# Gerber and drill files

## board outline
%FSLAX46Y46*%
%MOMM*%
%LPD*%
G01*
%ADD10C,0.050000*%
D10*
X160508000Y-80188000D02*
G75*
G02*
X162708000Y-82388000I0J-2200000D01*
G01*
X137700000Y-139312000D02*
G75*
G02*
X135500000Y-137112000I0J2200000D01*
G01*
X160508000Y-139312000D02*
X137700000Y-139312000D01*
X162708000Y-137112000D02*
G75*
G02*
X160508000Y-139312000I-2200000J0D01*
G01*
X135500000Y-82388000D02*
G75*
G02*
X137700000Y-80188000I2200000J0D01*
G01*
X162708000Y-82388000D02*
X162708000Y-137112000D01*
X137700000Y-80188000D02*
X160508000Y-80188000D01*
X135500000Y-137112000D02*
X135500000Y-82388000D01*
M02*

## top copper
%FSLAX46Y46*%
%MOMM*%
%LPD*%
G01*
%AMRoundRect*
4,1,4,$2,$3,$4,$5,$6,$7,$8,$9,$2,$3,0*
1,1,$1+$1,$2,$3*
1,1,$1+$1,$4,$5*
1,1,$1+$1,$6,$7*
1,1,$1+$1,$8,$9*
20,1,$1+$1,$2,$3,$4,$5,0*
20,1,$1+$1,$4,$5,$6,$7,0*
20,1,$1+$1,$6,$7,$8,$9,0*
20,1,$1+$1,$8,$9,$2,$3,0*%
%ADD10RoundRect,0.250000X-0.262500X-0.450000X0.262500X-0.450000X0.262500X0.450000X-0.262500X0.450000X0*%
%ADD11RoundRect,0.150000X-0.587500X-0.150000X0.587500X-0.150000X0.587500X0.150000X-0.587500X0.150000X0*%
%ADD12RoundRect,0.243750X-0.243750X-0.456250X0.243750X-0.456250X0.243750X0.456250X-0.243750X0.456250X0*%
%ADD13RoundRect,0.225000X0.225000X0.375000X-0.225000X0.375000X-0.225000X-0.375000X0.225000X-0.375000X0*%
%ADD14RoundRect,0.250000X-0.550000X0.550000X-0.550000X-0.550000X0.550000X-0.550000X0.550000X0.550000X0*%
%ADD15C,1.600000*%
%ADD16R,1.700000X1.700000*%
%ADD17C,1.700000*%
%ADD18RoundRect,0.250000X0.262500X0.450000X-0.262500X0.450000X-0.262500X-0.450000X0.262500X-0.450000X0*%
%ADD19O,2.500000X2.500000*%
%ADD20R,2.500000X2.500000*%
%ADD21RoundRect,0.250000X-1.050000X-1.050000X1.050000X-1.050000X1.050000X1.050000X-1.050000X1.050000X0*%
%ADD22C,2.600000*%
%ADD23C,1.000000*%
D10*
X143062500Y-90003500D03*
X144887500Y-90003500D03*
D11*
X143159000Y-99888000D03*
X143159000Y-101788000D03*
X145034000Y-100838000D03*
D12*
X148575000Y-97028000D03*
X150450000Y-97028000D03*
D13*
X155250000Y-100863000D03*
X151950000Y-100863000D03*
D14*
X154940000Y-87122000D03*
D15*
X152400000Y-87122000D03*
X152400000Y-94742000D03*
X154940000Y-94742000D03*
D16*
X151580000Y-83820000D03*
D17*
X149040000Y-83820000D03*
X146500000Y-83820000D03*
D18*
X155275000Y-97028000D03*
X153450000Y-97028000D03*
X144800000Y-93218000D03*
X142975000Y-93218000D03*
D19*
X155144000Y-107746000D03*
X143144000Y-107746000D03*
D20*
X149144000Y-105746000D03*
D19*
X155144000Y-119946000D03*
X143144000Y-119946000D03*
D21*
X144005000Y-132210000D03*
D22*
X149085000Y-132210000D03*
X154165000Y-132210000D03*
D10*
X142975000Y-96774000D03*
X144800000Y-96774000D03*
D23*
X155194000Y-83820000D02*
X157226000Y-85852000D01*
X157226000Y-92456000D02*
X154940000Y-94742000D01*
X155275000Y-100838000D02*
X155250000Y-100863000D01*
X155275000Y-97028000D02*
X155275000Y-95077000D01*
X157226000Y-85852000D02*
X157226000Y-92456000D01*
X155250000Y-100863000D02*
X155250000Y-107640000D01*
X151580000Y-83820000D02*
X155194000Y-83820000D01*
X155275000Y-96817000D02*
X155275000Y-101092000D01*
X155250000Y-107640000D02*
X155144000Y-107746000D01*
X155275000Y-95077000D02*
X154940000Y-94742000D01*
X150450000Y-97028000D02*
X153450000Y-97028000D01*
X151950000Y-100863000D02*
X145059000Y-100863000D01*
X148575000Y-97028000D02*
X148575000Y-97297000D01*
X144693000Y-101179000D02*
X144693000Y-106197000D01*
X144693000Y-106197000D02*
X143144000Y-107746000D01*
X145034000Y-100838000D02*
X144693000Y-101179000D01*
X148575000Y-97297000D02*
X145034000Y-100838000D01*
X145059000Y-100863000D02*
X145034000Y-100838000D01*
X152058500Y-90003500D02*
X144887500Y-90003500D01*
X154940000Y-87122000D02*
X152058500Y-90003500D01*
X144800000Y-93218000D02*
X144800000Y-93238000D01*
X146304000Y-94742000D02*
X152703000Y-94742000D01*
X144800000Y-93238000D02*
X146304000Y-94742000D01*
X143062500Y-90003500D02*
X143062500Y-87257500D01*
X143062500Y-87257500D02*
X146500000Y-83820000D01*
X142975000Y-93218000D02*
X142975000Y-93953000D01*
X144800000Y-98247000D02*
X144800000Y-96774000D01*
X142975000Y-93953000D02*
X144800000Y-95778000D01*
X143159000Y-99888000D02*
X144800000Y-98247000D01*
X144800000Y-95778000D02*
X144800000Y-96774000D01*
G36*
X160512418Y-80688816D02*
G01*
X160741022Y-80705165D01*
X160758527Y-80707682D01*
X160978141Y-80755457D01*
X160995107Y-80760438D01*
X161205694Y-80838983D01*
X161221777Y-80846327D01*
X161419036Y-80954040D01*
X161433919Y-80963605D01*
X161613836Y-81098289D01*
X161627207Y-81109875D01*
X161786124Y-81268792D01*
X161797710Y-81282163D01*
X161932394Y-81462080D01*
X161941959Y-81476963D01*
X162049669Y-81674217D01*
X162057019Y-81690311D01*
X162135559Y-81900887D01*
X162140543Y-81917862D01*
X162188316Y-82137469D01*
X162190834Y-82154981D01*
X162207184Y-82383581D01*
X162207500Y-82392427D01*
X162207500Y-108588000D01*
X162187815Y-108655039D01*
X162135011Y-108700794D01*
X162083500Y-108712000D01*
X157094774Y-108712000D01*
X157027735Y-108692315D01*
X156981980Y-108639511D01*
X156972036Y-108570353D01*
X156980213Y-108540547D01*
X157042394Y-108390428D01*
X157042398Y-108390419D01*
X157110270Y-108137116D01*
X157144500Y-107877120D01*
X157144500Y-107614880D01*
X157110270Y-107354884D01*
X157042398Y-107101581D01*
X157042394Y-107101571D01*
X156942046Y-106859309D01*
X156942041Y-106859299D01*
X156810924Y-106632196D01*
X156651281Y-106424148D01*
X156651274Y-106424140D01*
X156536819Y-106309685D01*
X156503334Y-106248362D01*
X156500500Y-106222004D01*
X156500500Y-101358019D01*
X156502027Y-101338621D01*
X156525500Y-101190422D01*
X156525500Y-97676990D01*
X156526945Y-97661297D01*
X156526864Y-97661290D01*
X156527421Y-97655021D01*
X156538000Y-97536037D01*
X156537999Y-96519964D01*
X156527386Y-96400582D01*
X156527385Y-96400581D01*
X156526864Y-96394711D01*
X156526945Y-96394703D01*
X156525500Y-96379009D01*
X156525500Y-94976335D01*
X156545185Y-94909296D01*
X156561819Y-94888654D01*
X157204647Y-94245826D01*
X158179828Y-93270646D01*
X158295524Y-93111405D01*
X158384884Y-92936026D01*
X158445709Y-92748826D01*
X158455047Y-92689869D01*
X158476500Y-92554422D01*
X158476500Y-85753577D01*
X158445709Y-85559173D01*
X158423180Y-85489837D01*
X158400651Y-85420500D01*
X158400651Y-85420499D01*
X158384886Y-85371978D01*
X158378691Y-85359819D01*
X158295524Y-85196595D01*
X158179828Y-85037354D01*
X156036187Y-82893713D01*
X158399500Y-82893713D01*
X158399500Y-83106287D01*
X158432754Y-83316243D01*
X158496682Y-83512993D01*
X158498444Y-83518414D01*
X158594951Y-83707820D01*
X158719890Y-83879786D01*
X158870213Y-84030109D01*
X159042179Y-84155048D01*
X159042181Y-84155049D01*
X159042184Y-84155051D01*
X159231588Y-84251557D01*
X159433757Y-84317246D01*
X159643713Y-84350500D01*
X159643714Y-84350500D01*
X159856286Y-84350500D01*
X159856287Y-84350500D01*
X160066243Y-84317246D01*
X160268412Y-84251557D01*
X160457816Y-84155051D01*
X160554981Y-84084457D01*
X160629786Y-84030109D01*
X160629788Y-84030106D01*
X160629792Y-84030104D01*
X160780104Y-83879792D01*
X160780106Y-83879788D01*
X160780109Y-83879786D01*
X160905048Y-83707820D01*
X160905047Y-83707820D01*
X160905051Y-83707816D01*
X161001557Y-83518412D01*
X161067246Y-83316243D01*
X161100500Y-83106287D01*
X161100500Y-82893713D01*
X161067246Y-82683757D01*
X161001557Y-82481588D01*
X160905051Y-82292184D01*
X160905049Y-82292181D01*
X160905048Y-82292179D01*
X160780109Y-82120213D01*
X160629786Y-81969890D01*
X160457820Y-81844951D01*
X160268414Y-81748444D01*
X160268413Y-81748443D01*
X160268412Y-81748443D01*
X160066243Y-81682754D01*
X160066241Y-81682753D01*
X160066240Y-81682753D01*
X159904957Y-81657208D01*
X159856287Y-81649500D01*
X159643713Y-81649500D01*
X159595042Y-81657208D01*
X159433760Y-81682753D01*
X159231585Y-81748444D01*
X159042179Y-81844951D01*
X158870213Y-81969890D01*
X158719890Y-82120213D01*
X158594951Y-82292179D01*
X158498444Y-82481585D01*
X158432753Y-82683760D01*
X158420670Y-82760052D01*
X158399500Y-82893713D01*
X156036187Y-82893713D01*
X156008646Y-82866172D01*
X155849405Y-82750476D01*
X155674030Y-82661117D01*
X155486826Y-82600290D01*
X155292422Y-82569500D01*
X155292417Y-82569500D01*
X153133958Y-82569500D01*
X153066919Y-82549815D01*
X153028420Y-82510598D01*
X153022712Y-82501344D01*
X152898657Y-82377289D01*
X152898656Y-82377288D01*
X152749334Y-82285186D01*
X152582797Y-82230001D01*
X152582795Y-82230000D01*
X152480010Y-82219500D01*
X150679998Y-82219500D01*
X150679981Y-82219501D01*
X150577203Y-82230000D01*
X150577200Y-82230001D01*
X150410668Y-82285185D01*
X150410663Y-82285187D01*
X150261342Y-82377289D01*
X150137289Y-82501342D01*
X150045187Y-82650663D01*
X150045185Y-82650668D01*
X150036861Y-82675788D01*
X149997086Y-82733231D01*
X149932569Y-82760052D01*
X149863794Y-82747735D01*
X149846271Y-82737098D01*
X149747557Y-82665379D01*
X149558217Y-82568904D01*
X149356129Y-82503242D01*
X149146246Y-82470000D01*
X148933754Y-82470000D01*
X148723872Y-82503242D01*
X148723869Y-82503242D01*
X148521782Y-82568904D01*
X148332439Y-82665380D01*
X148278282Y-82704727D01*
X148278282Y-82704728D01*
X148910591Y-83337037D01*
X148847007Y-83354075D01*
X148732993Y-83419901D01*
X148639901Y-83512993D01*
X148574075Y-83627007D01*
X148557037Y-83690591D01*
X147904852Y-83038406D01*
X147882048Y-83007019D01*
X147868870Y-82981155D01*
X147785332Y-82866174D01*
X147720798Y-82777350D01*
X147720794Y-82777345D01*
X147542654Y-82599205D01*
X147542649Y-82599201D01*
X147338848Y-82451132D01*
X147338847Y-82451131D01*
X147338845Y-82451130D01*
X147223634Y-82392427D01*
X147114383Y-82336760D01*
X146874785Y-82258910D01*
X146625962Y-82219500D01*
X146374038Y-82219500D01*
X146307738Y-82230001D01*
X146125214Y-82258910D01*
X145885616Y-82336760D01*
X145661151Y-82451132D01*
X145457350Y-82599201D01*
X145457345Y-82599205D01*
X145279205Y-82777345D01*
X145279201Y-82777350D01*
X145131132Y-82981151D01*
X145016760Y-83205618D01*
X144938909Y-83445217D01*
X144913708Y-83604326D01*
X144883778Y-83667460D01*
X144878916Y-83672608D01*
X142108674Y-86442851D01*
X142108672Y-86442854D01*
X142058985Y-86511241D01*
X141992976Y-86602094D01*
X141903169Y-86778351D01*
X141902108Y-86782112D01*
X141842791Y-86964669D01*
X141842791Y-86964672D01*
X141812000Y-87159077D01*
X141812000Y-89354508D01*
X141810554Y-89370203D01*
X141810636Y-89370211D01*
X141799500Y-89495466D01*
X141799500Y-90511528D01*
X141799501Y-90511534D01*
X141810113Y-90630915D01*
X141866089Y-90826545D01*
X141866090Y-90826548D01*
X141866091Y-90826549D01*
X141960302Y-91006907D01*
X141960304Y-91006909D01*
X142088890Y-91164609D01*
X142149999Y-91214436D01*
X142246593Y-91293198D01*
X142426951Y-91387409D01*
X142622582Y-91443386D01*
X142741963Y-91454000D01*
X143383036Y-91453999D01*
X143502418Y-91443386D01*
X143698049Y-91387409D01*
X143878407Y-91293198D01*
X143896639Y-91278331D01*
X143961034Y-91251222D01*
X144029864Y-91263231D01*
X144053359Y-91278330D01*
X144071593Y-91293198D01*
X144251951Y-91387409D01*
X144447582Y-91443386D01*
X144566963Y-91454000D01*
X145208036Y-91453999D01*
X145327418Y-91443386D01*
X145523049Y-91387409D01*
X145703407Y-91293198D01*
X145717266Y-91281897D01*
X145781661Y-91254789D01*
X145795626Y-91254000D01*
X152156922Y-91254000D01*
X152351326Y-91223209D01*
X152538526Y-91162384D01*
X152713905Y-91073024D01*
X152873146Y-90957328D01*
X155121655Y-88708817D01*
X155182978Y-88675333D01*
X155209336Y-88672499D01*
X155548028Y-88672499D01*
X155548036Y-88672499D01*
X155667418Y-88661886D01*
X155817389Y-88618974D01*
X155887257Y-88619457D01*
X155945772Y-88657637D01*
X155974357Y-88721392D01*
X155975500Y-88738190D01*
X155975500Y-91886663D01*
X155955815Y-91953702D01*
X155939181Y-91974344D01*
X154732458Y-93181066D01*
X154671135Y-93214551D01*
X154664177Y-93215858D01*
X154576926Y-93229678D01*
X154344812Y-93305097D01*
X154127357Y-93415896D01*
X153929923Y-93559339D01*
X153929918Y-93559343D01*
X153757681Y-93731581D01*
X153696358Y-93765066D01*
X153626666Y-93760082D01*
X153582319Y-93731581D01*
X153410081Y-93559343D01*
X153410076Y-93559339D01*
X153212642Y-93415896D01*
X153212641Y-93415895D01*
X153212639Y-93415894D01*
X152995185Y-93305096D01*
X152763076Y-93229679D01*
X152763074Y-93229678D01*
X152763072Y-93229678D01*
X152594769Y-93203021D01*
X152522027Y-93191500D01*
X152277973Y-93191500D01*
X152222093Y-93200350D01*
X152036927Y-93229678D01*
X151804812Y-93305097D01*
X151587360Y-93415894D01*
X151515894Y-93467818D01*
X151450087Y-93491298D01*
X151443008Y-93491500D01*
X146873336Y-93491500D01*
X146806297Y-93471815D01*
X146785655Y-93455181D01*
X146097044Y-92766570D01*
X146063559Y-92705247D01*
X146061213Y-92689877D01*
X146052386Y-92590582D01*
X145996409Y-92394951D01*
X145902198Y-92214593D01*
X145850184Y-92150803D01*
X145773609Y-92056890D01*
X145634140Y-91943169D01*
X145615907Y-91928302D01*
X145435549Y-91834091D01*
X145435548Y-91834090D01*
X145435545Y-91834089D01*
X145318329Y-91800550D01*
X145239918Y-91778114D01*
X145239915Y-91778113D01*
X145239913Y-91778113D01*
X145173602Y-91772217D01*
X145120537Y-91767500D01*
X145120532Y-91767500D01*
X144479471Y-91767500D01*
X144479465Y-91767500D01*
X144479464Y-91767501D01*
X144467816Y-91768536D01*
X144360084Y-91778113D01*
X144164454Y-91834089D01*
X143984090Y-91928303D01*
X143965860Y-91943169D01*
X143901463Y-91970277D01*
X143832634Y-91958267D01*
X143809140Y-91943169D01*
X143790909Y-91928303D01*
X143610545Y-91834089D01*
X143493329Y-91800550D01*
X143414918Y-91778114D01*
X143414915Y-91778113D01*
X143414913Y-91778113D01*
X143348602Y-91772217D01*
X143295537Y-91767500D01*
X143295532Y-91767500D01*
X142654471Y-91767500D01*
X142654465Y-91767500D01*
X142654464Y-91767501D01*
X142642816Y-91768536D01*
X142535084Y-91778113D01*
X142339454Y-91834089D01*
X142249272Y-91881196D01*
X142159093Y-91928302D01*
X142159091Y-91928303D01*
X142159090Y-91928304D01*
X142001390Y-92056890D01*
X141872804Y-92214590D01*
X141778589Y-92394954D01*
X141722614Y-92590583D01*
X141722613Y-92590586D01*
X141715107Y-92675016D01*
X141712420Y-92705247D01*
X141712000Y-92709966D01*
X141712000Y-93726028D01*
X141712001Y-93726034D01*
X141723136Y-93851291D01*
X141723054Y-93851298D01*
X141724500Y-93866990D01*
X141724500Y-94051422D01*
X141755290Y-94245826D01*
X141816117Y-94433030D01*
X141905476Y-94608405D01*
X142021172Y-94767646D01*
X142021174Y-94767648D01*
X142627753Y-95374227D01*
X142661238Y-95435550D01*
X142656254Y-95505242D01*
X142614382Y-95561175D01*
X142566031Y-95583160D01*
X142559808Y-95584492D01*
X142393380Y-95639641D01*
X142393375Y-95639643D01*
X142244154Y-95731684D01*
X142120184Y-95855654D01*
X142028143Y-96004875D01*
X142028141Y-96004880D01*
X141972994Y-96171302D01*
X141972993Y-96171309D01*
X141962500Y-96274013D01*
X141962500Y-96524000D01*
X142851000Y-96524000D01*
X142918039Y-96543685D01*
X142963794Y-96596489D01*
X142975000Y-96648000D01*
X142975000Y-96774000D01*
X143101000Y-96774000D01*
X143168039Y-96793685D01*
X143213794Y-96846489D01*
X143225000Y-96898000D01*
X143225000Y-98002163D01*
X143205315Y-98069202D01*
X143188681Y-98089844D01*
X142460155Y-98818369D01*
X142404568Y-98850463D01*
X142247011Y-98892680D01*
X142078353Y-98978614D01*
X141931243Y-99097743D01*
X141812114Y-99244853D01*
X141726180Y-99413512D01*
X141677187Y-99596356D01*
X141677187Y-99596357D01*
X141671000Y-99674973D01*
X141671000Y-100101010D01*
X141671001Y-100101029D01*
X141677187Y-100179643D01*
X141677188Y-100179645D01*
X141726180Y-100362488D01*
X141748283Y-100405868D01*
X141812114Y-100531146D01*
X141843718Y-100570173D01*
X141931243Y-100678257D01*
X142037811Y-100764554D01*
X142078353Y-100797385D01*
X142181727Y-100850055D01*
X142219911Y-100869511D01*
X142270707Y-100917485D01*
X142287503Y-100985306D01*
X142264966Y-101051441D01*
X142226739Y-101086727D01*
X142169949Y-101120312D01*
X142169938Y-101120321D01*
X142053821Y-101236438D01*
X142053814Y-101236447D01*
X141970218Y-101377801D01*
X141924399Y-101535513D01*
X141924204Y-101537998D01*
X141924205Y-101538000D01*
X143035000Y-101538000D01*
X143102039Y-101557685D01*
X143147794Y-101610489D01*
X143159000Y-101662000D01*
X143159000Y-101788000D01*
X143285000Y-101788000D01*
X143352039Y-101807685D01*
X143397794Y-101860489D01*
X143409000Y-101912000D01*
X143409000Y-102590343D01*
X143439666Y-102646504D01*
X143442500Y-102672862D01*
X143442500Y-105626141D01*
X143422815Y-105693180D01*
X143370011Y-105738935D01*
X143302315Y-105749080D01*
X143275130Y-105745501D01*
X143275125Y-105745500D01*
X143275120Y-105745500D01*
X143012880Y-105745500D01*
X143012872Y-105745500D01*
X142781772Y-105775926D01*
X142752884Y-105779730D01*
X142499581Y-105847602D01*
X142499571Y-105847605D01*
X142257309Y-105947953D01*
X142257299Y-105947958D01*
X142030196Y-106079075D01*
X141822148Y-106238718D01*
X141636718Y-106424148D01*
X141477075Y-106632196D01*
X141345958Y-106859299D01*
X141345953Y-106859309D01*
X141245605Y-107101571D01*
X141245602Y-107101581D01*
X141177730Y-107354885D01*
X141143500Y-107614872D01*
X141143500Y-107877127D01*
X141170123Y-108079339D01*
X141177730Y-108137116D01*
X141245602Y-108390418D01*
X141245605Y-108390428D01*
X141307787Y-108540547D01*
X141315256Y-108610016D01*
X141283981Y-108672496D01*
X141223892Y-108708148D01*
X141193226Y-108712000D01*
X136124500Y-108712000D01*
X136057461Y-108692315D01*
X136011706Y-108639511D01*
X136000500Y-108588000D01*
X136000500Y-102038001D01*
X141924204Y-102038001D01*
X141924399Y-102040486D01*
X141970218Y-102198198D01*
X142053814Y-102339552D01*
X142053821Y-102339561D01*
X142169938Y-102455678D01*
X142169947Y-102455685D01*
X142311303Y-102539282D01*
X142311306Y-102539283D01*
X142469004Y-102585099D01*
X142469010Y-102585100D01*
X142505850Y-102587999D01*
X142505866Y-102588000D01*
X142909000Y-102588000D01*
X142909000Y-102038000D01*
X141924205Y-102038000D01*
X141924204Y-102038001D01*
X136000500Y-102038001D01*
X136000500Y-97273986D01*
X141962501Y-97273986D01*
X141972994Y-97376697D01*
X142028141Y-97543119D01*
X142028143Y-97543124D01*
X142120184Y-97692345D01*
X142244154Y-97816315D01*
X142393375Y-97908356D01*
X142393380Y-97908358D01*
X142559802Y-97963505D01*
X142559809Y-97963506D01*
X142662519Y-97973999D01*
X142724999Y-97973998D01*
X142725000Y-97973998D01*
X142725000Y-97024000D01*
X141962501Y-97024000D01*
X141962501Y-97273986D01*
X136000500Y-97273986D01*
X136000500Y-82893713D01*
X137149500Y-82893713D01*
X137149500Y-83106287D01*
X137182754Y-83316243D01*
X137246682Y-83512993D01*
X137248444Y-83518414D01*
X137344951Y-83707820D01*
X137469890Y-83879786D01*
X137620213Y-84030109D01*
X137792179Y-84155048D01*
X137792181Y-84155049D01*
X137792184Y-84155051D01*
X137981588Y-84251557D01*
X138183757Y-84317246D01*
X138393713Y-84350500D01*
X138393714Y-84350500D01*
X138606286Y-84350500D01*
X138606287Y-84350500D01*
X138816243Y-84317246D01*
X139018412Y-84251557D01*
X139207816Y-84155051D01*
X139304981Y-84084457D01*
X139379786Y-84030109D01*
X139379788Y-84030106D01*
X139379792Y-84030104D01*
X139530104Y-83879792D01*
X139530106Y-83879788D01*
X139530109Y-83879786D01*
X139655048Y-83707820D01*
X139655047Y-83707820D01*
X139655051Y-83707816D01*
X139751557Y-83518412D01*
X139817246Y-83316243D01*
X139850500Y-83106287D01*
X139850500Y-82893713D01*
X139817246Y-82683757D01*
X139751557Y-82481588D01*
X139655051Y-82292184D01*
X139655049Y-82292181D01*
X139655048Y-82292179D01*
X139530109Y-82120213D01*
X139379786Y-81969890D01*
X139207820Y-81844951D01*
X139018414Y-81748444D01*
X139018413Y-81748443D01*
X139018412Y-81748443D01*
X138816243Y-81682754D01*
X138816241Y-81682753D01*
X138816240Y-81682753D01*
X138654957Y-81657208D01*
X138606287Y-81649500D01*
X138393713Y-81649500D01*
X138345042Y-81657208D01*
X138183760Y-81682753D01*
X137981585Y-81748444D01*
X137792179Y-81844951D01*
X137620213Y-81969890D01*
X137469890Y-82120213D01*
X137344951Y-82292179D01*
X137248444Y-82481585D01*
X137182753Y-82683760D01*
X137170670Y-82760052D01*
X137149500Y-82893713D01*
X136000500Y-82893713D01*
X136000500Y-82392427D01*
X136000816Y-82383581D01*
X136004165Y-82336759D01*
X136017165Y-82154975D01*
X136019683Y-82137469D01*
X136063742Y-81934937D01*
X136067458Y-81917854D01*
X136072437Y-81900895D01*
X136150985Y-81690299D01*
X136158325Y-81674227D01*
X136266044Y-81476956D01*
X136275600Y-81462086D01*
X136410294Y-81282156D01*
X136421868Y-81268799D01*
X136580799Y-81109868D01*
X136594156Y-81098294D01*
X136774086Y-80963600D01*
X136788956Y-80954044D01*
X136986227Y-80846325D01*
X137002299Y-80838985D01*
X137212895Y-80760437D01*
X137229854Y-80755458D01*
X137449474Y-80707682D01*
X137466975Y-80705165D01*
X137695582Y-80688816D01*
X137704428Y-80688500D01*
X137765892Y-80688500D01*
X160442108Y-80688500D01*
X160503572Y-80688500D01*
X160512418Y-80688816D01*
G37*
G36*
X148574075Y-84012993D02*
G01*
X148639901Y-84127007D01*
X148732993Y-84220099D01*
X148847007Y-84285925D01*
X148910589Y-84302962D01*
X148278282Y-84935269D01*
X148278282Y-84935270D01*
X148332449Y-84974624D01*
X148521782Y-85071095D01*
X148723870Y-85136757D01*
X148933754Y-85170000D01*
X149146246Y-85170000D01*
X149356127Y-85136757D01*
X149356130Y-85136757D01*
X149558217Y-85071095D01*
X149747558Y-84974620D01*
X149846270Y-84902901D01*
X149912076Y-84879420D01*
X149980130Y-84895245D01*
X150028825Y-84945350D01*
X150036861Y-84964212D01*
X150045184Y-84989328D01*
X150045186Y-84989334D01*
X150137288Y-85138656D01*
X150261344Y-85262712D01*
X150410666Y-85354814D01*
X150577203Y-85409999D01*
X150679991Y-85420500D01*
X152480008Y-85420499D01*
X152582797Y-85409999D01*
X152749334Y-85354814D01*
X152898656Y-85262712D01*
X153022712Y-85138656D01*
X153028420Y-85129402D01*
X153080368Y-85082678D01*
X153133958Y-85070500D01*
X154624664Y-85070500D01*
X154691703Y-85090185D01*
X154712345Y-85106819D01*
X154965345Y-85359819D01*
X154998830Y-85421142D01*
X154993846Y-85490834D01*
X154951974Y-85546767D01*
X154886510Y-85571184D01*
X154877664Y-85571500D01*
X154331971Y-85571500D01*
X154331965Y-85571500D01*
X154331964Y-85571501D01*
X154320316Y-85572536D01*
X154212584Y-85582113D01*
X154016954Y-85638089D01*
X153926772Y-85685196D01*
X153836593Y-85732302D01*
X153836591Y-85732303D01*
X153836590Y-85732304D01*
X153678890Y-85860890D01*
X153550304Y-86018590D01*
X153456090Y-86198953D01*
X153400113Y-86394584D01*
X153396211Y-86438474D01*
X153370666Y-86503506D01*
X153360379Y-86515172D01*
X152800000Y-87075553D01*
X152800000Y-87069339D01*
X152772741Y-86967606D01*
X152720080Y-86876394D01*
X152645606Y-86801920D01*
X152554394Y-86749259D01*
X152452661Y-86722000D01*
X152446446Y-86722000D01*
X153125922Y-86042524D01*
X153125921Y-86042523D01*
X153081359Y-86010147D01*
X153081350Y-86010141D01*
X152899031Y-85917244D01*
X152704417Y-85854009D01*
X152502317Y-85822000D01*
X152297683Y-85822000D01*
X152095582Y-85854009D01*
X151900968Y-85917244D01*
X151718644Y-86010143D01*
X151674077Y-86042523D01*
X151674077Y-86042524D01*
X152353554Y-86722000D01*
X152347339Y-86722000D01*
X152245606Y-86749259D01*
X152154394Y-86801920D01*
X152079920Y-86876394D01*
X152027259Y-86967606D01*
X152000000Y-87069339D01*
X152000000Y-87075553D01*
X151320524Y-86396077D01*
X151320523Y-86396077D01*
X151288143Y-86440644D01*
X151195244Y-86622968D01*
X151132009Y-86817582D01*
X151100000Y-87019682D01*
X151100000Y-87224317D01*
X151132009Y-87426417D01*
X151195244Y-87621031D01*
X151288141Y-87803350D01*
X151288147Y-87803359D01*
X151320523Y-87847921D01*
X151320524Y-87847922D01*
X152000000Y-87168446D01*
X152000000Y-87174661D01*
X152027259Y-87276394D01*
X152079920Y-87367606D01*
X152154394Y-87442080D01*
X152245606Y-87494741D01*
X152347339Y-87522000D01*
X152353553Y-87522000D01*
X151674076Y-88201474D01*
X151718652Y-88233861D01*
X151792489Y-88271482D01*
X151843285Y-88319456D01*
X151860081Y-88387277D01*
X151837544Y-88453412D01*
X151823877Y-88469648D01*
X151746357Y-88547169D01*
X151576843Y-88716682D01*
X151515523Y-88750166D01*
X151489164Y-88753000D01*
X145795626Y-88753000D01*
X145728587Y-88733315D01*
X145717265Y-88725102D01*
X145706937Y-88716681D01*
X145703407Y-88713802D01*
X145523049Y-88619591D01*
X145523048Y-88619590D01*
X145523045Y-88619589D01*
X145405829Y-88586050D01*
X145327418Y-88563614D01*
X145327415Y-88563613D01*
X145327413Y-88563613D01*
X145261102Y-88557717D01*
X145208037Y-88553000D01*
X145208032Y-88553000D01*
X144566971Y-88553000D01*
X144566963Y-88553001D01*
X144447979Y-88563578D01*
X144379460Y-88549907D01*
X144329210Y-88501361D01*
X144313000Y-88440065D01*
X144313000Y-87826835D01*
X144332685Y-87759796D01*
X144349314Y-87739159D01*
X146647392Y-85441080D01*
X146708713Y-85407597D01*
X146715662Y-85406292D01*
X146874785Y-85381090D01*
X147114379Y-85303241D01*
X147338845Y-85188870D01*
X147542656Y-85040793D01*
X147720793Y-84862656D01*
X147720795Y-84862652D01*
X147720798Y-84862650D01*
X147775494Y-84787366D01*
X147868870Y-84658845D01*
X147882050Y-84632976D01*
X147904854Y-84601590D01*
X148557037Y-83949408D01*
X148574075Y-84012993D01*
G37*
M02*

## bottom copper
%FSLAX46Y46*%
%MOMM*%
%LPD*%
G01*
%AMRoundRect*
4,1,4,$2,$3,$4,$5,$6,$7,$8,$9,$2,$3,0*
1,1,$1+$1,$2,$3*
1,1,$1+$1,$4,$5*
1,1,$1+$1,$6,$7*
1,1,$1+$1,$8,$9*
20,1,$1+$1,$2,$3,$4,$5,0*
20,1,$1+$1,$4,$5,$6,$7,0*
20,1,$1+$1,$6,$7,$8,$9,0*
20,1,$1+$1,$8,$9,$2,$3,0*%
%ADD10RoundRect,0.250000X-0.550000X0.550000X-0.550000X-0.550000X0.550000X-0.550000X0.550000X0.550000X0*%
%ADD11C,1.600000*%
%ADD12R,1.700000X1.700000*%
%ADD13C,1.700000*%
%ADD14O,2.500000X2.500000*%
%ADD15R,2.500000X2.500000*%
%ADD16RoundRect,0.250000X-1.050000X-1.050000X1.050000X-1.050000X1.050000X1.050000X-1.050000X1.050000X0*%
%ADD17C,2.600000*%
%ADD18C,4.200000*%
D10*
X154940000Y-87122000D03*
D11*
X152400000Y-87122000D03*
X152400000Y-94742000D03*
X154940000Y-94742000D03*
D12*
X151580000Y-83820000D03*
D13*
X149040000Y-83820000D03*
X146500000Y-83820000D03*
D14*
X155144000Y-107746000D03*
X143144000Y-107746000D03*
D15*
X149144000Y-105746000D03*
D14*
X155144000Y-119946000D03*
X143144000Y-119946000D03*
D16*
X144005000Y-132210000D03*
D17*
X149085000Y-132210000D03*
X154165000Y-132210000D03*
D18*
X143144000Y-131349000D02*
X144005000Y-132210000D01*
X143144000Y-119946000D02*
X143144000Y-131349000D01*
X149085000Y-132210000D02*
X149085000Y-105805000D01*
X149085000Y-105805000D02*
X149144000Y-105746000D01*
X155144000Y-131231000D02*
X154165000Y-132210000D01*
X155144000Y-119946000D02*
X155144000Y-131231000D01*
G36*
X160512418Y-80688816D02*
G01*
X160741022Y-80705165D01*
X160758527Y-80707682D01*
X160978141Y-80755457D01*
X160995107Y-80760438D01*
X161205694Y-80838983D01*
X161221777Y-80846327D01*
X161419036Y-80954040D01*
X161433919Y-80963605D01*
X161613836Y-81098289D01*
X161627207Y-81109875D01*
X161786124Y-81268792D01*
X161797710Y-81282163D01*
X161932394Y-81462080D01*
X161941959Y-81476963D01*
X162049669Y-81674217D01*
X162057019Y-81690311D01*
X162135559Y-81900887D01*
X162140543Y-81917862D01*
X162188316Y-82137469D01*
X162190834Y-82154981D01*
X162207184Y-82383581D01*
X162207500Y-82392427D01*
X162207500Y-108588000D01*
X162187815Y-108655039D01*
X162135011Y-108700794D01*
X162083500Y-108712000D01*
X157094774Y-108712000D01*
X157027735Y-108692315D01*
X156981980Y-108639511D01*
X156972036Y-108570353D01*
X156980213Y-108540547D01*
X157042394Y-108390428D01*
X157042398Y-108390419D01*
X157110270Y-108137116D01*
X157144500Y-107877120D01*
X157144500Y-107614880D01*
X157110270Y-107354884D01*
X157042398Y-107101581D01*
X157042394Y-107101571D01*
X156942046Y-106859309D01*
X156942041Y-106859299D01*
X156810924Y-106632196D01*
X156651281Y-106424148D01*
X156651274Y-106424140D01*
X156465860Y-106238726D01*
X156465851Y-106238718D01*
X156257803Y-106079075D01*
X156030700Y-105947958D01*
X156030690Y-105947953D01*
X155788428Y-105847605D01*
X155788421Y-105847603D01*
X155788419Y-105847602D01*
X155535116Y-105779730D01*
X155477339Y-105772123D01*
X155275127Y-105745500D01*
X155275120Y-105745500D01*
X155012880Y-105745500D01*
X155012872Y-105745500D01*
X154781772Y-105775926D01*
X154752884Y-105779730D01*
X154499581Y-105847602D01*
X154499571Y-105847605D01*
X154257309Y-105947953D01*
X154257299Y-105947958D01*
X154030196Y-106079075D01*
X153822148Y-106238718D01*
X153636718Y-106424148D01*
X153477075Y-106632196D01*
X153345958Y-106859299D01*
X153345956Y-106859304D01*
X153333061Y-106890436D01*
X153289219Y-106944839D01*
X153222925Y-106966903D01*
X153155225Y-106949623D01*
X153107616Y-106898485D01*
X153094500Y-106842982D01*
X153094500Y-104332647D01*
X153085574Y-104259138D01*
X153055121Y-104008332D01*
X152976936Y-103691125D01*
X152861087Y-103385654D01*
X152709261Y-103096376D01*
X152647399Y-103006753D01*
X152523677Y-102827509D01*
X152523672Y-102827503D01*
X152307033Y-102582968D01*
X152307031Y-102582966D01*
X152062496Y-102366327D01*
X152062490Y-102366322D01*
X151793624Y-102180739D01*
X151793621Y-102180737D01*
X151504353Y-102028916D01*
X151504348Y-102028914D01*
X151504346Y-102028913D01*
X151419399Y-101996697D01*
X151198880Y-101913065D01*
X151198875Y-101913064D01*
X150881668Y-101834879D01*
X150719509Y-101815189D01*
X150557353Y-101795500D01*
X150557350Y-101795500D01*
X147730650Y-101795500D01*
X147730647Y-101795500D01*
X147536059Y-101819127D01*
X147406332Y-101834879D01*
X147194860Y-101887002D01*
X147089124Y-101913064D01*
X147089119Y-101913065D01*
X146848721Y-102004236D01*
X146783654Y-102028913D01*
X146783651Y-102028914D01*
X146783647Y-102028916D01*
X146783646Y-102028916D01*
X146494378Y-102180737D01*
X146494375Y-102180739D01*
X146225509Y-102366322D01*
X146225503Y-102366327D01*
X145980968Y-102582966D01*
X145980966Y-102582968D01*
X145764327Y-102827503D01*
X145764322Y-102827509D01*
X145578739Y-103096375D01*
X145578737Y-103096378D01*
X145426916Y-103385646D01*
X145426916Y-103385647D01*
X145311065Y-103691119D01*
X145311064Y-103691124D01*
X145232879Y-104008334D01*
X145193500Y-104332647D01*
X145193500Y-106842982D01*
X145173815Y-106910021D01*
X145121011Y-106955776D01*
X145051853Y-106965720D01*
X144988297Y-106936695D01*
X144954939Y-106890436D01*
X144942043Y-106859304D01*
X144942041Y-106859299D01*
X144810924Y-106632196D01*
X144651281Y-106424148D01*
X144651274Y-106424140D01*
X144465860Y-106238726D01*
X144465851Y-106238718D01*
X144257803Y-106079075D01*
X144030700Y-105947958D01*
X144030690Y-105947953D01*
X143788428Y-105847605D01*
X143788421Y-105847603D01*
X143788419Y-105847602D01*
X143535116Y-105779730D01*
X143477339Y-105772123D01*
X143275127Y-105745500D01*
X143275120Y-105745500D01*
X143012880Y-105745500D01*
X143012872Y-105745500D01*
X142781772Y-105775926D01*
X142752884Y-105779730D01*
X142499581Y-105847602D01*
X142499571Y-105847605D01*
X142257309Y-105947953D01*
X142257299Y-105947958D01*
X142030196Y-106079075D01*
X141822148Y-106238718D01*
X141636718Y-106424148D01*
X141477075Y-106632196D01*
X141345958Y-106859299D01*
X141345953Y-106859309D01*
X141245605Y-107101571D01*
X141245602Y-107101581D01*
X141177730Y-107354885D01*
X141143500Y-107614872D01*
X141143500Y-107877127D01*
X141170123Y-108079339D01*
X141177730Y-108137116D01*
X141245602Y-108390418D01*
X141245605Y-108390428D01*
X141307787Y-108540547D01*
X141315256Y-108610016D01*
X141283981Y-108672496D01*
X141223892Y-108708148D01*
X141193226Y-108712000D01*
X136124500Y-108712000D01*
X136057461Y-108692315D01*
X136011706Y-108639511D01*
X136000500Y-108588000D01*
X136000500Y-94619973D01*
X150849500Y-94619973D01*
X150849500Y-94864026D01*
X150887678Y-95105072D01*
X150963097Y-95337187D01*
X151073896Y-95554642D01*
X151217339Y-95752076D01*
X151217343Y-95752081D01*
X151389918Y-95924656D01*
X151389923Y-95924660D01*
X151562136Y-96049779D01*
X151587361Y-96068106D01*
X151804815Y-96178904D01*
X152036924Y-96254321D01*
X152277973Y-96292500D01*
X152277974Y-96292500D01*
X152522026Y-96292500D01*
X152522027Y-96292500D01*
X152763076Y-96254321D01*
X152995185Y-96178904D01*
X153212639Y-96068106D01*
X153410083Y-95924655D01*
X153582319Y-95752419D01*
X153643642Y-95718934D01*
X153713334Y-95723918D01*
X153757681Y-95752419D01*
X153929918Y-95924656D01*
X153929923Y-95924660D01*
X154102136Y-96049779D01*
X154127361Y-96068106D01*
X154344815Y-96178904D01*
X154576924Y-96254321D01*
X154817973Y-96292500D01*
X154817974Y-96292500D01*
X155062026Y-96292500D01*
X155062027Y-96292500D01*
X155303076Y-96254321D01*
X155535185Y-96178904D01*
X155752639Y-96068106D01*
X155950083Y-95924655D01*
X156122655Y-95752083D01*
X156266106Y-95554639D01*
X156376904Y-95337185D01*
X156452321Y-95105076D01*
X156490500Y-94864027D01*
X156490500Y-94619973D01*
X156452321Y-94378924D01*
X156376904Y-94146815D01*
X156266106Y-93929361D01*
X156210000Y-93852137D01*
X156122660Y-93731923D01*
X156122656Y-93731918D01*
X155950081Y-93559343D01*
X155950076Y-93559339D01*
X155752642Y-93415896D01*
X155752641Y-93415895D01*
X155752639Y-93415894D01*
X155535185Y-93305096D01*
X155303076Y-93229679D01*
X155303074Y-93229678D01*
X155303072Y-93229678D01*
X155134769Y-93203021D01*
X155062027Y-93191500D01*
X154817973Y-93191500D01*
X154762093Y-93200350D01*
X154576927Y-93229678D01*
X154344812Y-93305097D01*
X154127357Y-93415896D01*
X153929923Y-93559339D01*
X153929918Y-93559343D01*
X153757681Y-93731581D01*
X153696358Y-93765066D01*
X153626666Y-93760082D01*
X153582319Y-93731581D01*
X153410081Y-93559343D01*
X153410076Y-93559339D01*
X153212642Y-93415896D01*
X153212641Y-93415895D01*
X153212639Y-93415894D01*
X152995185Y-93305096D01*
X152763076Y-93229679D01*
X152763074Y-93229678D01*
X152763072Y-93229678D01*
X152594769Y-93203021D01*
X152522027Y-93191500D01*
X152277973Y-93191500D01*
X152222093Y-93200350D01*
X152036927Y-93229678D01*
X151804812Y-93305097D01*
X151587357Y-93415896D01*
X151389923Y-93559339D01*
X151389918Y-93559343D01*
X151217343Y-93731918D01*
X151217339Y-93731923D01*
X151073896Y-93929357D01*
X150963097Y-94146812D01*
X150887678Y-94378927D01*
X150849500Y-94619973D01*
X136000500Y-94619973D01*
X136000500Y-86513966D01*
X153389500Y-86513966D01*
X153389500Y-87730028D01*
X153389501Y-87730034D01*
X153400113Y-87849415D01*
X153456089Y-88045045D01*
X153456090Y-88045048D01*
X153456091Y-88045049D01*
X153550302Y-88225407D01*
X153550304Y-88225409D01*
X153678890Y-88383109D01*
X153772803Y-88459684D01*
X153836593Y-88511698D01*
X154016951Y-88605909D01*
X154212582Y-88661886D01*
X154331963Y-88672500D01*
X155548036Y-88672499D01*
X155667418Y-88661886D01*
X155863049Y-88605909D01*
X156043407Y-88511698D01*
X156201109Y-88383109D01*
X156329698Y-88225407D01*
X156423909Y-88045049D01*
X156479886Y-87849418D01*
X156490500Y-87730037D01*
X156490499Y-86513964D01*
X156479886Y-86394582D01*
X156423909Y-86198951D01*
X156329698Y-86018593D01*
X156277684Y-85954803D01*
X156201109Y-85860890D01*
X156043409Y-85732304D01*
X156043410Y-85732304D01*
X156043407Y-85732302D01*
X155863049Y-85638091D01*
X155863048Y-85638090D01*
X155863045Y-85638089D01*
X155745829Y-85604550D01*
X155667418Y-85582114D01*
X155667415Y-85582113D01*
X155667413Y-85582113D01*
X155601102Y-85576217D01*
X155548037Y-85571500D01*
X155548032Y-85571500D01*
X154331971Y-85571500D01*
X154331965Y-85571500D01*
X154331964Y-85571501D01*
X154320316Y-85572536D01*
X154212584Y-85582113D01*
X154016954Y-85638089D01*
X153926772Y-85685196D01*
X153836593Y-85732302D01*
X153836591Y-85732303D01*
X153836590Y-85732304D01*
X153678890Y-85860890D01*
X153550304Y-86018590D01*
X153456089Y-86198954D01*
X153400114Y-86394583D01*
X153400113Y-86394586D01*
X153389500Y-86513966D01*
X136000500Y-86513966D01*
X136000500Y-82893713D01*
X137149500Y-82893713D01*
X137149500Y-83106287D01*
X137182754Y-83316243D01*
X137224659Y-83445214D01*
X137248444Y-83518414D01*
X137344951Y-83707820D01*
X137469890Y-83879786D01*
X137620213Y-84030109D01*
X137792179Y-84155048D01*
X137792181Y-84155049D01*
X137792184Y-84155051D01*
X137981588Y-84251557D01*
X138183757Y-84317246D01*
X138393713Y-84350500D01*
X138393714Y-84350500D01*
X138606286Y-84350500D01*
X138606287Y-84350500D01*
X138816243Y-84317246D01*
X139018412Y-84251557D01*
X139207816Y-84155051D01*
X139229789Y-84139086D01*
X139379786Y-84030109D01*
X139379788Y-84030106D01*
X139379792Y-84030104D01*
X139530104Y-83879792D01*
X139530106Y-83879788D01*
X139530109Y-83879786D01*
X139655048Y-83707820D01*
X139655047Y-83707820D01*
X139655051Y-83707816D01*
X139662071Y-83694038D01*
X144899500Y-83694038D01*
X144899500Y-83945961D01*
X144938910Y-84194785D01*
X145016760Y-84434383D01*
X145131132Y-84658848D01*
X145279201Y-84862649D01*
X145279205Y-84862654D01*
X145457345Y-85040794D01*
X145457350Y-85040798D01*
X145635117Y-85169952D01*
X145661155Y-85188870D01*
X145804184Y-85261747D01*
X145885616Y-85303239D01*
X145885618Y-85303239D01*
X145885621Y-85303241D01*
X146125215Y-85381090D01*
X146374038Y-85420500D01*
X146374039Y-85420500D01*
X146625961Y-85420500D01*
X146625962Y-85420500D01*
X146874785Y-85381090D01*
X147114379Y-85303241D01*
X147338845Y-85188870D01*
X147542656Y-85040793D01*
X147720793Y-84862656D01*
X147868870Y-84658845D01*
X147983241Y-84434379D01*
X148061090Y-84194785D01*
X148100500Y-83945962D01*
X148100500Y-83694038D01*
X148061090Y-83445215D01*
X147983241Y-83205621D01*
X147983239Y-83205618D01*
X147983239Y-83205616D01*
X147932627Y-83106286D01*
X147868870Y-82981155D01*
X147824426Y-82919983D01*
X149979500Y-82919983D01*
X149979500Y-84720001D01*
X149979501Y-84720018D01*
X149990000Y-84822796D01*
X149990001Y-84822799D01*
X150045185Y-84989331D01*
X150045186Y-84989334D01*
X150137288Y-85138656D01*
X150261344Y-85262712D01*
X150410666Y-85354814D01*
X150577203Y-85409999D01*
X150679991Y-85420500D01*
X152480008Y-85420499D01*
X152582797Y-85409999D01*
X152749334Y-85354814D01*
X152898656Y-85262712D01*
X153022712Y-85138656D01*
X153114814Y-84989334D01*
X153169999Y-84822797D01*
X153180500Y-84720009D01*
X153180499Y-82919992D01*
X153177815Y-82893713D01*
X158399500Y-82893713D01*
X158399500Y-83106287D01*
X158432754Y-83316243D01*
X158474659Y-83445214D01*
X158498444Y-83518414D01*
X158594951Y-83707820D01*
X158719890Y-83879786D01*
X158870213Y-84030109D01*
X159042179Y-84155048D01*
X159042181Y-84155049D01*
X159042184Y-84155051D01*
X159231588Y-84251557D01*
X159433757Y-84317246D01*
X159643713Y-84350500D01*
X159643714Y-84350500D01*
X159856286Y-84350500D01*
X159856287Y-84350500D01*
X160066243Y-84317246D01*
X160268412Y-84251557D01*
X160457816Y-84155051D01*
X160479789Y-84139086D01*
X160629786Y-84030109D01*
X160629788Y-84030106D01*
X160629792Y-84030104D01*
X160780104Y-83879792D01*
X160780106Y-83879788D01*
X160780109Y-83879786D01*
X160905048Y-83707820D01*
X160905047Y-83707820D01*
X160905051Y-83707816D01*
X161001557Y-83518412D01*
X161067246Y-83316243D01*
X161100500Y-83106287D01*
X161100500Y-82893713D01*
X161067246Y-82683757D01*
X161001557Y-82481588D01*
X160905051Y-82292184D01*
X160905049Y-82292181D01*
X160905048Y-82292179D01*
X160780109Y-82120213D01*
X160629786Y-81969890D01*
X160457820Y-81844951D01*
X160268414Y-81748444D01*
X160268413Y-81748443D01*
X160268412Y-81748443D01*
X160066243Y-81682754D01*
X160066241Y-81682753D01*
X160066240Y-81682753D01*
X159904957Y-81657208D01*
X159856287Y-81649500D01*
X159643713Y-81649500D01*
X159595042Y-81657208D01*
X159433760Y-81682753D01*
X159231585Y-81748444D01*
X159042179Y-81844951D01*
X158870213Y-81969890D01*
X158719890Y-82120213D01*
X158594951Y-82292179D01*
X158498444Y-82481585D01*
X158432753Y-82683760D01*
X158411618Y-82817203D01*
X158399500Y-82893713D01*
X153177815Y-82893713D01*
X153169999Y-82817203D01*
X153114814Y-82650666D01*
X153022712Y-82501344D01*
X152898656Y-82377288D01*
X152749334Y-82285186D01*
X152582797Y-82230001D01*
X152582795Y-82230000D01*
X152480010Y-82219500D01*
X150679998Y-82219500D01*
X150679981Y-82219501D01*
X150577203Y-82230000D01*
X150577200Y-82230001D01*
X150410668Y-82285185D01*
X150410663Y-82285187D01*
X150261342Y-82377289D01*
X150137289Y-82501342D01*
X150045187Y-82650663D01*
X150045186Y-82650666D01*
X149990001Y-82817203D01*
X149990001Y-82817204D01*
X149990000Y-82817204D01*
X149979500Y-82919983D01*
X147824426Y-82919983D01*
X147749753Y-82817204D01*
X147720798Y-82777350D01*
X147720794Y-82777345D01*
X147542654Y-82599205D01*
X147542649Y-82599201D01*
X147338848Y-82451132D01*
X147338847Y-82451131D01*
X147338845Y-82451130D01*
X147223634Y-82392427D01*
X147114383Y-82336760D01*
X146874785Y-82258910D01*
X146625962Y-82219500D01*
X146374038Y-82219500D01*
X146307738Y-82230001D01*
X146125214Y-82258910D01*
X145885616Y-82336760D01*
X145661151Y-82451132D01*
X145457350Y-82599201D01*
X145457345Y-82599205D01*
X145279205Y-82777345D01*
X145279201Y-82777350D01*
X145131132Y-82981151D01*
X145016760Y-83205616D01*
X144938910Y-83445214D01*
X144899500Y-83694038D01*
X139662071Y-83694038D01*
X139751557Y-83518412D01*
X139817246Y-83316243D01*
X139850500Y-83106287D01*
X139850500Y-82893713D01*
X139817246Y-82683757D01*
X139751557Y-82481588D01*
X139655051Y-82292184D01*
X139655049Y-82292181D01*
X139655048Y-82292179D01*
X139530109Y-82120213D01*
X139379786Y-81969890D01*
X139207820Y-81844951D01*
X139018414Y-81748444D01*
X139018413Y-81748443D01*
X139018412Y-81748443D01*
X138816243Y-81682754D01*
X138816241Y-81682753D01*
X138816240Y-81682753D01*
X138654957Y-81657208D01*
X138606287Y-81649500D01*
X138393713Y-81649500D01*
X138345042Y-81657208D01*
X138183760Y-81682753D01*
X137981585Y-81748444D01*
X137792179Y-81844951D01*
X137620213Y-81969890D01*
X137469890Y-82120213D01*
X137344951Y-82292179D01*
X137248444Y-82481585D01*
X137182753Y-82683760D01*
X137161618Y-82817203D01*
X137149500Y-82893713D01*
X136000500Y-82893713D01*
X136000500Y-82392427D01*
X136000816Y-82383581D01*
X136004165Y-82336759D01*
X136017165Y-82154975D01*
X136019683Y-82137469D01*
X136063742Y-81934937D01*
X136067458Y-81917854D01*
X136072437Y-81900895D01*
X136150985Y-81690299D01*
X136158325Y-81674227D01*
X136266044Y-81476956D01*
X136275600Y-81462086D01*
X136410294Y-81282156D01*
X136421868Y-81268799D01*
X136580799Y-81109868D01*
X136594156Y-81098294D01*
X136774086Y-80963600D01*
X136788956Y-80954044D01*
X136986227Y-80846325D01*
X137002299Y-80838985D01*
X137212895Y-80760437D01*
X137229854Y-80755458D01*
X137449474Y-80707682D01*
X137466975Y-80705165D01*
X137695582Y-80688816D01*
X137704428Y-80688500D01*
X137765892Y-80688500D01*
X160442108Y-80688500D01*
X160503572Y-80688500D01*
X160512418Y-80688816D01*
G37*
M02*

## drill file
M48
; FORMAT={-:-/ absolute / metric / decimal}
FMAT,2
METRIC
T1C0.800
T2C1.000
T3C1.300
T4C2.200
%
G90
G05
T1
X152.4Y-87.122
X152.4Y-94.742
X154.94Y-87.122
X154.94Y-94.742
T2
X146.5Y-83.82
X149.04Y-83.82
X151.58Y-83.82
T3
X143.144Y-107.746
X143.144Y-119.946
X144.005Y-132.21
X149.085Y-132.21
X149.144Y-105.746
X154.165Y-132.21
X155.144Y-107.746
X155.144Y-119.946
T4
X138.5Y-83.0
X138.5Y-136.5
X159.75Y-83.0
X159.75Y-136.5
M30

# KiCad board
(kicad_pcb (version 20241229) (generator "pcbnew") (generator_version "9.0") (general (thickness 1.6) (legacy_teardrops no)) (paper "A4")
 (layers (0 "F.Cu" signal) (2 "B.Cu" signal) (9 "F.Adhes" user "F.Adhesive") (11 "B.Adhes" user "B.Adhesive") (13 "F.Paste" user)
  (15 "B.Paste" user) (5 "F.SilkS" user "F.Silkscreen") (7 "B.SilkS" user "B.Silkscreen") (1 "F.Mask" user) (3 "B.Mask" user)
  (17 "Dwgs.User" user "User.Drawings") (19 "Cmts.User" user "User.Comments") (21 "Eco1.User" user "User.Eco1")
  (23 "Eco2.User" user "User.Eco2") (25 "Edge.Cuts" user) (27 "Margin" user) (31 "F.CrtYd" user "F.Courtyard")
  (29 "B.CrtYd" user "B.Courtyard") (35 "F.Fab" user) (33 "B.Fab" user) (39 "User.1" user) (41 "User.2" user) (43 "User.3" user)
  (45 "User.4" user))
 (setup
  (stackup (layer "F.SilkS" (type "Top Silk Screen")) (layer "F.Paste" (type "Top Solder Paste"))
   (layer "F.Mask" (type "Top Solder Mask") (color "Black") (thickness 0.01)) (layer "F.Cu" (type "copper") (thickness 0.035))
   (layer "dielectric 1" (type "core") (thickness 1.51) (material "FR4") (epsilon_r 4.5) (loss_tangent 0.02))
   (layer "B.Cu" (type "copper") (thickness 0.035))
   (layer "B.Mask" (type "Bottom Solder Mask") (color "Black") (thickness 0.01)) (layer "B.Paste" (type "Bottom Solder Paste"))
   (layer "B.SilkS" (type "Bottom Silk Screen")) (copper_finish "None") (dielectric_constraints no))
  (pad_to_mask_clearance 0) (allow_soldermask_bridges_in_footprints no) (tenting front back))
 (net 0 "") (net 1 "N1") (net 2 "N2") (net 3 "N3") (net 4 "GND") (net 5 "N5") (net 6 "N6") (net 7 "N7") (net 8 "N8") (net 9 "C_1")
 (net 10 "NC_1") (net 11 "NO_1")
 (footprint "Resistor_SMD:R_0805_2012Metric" (layer "F.Cu") (at 143.975 90.0035)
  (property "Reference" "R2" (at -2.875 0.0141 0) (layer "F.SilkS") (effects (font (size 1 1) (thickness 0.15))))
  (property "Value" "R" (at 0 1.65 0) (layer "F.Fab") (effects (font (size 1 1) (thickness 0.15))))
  (pad "1" smd roundrect (at -0.9125 0) (size 1.025 1.4) (layers "F.Cu" "F.Mask" "F.Paste") (roundrect_rratio 0.243902) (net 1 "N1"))
  (pad "2" smd roundrect (at 0.9125 0) (size 1.025 1.4) (layers "F.Cu" "F.Mask" "F.Paste") (roundrect_rratio 0.243902) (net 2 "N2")))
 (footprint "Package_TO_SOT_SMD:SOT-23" (layer "F.Cu") (at 144.0965 100.838)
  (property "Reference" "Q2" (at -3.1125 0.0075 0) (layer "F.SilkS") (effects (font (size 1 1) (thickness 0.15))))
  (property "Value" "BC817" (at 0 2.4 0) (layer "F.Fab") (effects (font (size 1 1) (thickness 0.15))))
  (pad "1" smd roundrect (at -0.9375 -0.95) (size 1.475 0.6) (layers "F.Cu" "F.Mask" "F.Paste") (roundrect_rratio 0.25) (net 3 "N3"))
  (pad "2" smd roundrect (at -0.9375 0.95) (size 1.475 0.6) (layers "F.Cu" "F.Mask" "F.Paste") (roundrect_rratio 0.25) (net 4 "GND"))
  (pad "3" smd roundrect (at 0.9375 0) (size 1.475 0.6) (layers "F.Cu" "F.Mask" "F.Paste") (roundrect_rratio 0.25) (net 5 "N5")))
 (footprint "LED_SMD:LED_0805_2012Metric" (layer "F.Cu") (at 149.5125 97.028)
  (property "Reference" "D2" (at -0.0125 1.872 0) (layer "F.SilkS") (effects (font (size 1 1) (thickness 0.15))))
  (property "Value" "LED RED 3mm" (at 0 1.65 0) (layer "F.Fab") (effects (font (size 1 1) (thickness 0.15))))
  (pad "1" smd roundrect (at -0.9375 0) (size 0.975 1.4) (layers "F.Cu" "F.Mask" "F.Paste") (roundrect_rratio 0.25) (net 5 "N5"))
  (pad "2" smd roundrect (at 0.9375 0) (size 0.975 1.4) (layers "F.Cu" "F.Mask" "F.Paste") (roundrect_rratio 0.25) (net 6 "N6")))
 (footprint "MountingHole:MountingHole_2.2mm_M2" (layer "F.Cu") (at 138.5 83)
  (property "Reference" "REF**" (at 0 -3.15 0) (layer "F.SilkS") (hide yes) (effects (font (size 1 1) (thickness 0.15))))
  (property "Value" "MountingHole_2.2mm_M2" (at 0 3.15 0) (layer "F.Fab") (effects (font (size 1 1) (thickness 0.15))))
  (pad "" np_thru_hole circle (at 0 0) (size 2.2 2.2) (drill 2.2) (layers "*.Cu" "*.Mask")))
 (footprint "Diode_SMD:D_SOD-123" (layer "F.Cu") (at 153.6 100.863 180)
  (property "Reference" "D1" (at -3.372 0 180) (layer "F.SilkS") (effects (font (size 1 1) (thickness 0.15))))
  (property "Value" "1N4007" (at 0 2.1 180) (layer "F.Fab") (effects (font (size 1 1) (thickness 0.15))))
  (pad "1" smd roundrect (at -1.65 0 180) (size 0.9 1.2) (layers "F.Cu" "F.Mask" "F.Paste") (roundrect_rratio 0.25) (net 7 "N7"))
  (pad "2" smd roundrect (at 1.65 0 180) (size 0.9 1.2) (layers "F.Cu" "F.Mask" "F.Paste") (roundrect_rratio 0.25) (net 5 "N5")))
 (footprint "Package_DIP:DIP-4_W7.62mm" (layer "F.Cu") (at 154.94 87.122 -90)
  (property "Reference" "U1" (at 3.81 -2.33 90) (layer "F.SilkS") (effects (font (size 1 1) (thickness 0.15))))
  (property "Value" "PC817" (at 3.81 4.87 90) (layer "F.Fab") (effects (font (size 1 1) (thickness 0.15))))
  (pad "1" thru_hole roundrect (at 0 0 270) (size 1.6 1.6) (drill 0.8) (layers "*.Cu" "*.Mask") (remove_unused_layers no)
   (roundrect_rratio 0.15625) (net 2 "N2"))
  (pad "2" thru_hole circle (at 0 2.54 270) (size 1.6 1.6) (drill 0.8) (layers "*.Cu" "*.Mask") (remove_unused_layers no) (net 4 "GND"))
  (pad "3" thru_hole circle (at 7.62 2.54 270) (size 1.6 1.6) (drill 0.8) (layers "*.Cu" "*.Mask") (remove_unused_layers no) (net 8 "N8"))
  (pad "4" thru_hole circle (at 7.62 0 270) (size 1.6 1.6) (drill 0.8) (layers "*.Cu" "*.Mask") (remove_unused_layers no) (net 7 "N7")))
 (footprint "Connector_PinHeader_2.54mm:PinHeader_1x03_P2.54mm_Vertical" (layer "F.Cu") (at 151.58 83.82 -90)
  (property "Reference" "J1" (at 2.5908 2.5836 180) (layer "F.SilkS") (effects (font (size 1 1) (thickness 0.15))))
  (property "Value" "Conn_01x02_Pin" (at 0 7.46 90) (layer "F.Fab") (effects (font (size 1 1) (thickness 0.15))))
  (pad "1" thru_hole rect (at 0 0 270) (size 1.7 1.7) (drill 1) (layers "*.Cu" "*.Mask") (remove_unused_layers no) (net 7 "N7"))
  (pad "2" thru_hole circle (at 0 2.54 270) (size 1.7 1.7) (drill 1) (layers "*.Cu" "*.Mask") (remove_unused_layers no) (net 4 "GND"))
  (pad "3" thru_hole circle (at 0 5.08 270) (size 1.7 1.7) (drill 1) (layers "*.Cu" "*.Mask") (remove_unused_layers no) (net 1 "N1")))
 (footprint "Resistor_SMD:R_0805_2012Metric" (layer "F.Cu") (at 154.3625 97.028 180)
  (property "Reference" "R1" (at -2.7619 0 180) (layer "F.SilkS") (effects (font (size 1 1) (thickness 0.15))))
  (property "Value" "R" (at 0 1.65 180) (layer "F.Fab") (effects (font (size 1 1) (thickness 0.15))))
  (pad "1" smd roundrect (at -0.9125 0 180) (size 1.025 1.4) (layers "F.Cu" "F.Mask" "F.Paste") (roundrect_rratio 0.243902) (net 7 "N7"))
  (pad "2" smd roundrect (at 0.9125 0 180) (size 1.025 1.4) (layers "F.Cu" "F.Mask" "F.Paste") (roundrect_rratio 0.243902) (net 6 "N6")))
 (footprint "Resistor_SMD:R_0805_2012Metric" (layer "F.Cu") (at 143.8875 93.218 180)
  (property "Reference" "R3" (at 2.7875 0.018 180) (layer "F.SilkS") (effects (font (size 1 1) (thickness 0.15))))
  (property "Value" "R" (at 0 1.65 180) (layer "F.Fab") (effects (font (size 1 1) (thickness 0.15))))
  (pad "1" smd roundrect (at -0.9125 0 180) (size 1.025 1.4) (layers "F.Cu" "F.Mask" "F.Paste") (roundrect_rratio 0.243902) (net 8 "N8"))
  (pad "2" smd roundrect (at 0.9125 0 180) (size 1.025 1.4) (layers "F.Cu" "F.Mask" "F.Paste") (roundrect_rratio 0.243902) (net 3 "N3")))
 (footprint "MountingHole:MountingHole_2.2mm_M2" (layer "F.Cu") (at 159.75 83)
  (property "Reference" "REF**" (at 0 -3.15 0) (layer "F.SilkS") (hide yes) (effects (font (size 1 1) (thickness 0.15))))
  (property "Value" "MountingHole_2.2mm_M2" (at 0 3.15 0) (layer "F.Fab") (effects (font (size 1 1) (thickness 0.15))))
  (pad "" np_thru_hole circle (at 0 0) (size 2.2 2.2) (drill 2.2) (layers "*.Cu" "*.Mask")))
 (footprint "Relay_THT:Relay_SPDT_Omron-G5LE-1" (layer "F.Cu") (at 149.144 105.746)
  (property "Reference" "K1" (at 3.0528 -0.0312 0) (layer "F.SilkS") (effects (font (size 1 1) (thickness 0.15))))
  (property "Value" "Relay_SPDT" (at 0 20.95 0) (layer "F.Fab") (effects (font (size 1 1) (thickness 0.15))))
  (pad "1" thru_hole oval (at 6 2) (size 2.5 2.5) (drill 1.3) (layers "*.Cu" "*.Mask") (remove_unused_layers no) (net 7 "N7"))
  (pad "2" thru_hole oval (at -6 2) (size 2.5 2.5) (drill 1.3) (layers "*.Cu" "*.Mask") (remove_unused_layers no) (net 5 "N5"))
  (pad "3" thru_hole rect (at 0 0) (size 2.5 2.5) (drill 1.3) (layers "*.Cu" "*.Mask") (remove_unused_layers no) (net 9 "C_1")
   (clearance 2.7))
  (pad "4" thru_hole oval (at 6 14.2) (size 2.5 2.5) (drill 1.3) (layers "*.Cu" "*.Mask") (remove_unused_layers no) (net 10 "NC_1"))
  (pad "5" thru_hole oval (at -6 14.2) (size 2.5 2.5) (drill 1.3) (layers "*.Cu" "*.Mask") (remove_unused_layers no) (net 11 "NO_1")))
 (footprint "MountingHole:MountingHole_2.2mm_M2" (layer "F.Cu") (at 138.5 136.5)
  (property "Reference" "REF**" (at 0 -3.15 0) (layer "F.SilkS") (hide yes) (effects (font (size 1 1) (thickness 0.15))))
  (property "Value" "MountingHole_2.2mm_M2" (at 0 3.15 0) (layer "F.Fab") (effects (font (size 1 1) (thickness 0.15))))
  (pad "" np_thru_hole circle (at 0 0) (size 2.2 2.2) (drill 2.2) (layers "*.Cu" "*.Mask")))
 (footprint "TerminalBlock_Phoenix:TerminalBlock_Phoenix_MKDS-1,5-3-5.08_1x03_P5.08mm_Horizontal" (layer "F.Cu") (at 144.005 132.21)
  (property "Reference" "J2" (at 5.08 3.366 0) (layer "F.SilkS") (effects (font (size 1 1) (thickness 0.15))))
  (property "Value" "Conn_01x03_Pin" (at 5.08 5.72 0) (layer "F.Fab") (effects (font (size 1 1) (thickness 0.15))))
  (pad "1" thru_hole roundrect (at 0 0) (size 2.6 2.6) (drill 1.3) (layers "*.Cu" "*.Mask") (remove_unused_layers no)
   (roundrect_rratio 0.096154) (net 11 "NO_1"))
  (pad "2" thru_hole circle (at 5.08 0) (size 2.6 2.6) (drill 1.3) (layers "*.Cu" "*.Mask") (remove_unused_layers no) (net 9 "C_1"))
  (pad "3" thru_hole circle (at 10.16 0) (size 2.6 2.6) (drill 1.3) (layers "*.Cu" "*.Mask") (remove_unused_layers no) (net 10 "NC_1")))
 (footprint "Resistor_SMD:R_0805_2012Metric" (layer "F.Cu") (at 143.8875 96.774)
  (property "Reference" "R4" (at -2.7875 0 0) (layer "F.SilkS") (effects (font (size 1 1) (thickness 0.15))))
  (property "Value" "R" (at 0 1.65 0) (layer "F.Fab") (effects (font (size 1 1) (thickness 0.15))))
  (pad "1" smd roundrect (at -0.9125 0) (size 1.025 1.4) (layers "F.Cu" "F.Mask" "F.Paste") (roundrect_rratio 0.243902) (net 4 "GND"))
  (pad "2" smd roundrect (at 0.9125 0) (size 1.025 1.4) (layers "F.Cu" "F.Mask" "F.Paste") (roundrect_rratio 0.243902) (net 3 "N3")))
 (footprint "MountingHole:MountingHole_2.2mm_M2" (layer "F.Cu") (at 159.75 136.5)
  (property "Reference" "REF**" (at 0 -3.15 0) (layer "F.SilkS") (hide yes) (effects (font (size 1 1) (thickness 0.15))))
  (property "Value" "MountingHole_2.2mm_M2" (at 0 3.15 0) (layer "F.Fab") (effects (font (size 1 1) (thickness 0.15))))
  (pad "" np_thru_hole circle (at 0 0) (size 2.2 2.2) (drill 2.2) (layers "*.Cu" "*.Mask")))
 (gr_arc (start 160.508 80.188) (mid 162.063635 80.832365) (end 162.708 82.388) (stroke (width 0.05) (type default)) (layer "Edge.Cuts"))
 (gr_arc (start 137.7 139.312) (mid 136.144365 138.667635) (end 135.5 137.112) (stroke (width 0.05) (type default)) (layer "Edge.Cuts"))
 (gr_line (start 160.508 139.312) (end 137.7 139.312) (stroke (width 0.05) (type default)) (layer "Edge.Cuts"))
 (gr_arc (start 162.708 137.112) (mid 162.063635 138.667635) (end 160.508 139.312) (stroke (width 0.05) (type default)) (layer "Edge.Cuts"))
 (gr_arc (start 135.5 82.388) (mid 136.144365 80.832365) (end 137.7 80.188) (stroke (width 0.05) (type default)) (layer "Edge.Cuts"))
 (gr_line (start 162.708 82.388) (end 162.708 137.112) (stroke (width 0.05) (type default)) (layer "Edge.Cuts"))
 (gr_line (start 137.7 80.188) (end 160.508 80.188) (stroke (width 0.05) (type default)) (layer "Edge.Cuts"))
 (gr_line (start 135.5 137.112) (end 135.5 82.388) (stroke (width 0.05) (type default)) (layer "Edge.Cuts"))
 (segment (start 155.194 83.82) (end 157.226 85.852) (width 1) (layer "F.Cu") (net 7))
 (segment (start 157.226 92.456) (end 154.94 94.742) (width 1) (layer "F.Cu") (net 7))
 (segment (start 155.275 100.838) (end 155.25 100.863) (width 1) (layer "F.Cu") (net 7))
 (segment (start 155.275 97.028) (end 155.275 95.077) (width 1) (layer "F.Cu") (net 7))
 (segment (start 157.226 85.852) (end 157.226 92.456) (width 1) (layer "F.Cu") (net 7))
 (segment (start 155.25 100.863) (end 155.25 107.64) (width 1) (layer "F.Cu") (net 7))
 (segment (start 151.58 83.82) (end 155.194 83.82) (width 1) (layer "F.Cu") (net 7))
 (segment (start 155.275 96.817) (end 155.275 101.092) (width 1) (layer "F.Cu") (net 7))
 (segment (start 155.25 107.64) (end 155.144 107.746) (width 1) (layer "F.Cu") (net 7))
 (segment (start 155.275 95.077) (end 154.94 94.742) (width 1) (layer "F.Cu") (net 7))
 (segment (start 143.144 131.349) (end 144.005 132.21) (width 4.2) (layer "B.Cu") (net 11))
 (segment (start 143.144 119.946) (end 143.144 131.349) (width 4.2) (layer "B.Cu") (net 11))
 (segment (start 149.085 132.21) (end 149.085 105.805) (width 4.2) (layer "B.Cu") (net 9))
 (segment (start 149.085 105.805) (end 149.144 105.746) (width 4.2) (layer "B.Cu") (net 9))
 (segment (start 155.144 131.231) (end 154.165 132.21) (width 4.2) (layer "B.Cu") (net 10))
 (segment (start 155.144 119.946) (end 155.144 131.231) (width 4.2) (layer "B.Cu") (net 10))
 (segment (start 150.45 97.028) (end 153.45 97.028) (width 1) (layer "F.Cu") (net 6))
 (segment (start 151.95 100.863) (end 145.059 100.863) (width 1) (layer "F.Cu") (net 5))
 (segment (start 148.575 97.028) (end 148.575 97.297) (width 1) (layer "F.Cu") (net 5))
 (segment (start 144.693 101.179) (end 144.693 106.197) (width 1) (layer "F.Cu") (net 5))
 (segment (start 144.693 106.197) (end 143.144 107.746) (width 1) (layer "F.Cu") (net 5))
 (segment (start 145.034 100.838) (end 144.693 101.179) (width 1) (layer "F.Cu") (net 5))
 (segment (start 148.575 97.297) (end 145.034 100.838) (width 1) (layer "F.Cu") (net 5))
 (segment (start 145.059 100.863) (end 145.034 100.838) (width 1) (layer "F.Cu") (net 5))
 (segment (start 152.0585 90.0035) (end 144.8875 90.0035) (width 1) (layer "F.Cu") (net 2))
 (segment (start 154.94 87.122) (end 152.0585 90.0035) (width 1) (layer "F.Cu") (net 2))
 (segment (start 144.8 93.218) (end 144.8 93.238) (width 1) (layer "F.Cu") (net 8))
 (segment (start 146.304 94.742) (end 152.703 94.742) (width 1) (layer "F.Cu") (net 8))
 (segment (start 144.8 93.238) (end 146.304 94.742) (width 1) (layer "F.Cu") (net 8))
 (segment (start 143.0625 90.0035) (end 143.0625 87.2575) (width 1) (layer "F.Cu") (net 1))
 (segment (start 143.0625 87.2575) (end 146.5 83.82) (width 1) (layer "F.Cu") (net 1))
 (segment (start 142.975 93.218) (end 142.975 93.953) (width 1) (layer "F.Cu") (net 3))
 (segment (start 144.8 98.247) (end 144.8 96.774) (width 1) (layer "F.Cu") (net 3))
 (segment (start 142.975 93.953) (end 144.8 95.778) (width 1) (layer "F.Cu") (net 3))
 (segment (start 143.159 99.888) (end 144.8 98.247) (width 1) (layer "F.Cu") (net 3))
 (segment (start 144.8 95.778) (end 144.8 96.774) (width 1) (layer "F.Cu") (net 3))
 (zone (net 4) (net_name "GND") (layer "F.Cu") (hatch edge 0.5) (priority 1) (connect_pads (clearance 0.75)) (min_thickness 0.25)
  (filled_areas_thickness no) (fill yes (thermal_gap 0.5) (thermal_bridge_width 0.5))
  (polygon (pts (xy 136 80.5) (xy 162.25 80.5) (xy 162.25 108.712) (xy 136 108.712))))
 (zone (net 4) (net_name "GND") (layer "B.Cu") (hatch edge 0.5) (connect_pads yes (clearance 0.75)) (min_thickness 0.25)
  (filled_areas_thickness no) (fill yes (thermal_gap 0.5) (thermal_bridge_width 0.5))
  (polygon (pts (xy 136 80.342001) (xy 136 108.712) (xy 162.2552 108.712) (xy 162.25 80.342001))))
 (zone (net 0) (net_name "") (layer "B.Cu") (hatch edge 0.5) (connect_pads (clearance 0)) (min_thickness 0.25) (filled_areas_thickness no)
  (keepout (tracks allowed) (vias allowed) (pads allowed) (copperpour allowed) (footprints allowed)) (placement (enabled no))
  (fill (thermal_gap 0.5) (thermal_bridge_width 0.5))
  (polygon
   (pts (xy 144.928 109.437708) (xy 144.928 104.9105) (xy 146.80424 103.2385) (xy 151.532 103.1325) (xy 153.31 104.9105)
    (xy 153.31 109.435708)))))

